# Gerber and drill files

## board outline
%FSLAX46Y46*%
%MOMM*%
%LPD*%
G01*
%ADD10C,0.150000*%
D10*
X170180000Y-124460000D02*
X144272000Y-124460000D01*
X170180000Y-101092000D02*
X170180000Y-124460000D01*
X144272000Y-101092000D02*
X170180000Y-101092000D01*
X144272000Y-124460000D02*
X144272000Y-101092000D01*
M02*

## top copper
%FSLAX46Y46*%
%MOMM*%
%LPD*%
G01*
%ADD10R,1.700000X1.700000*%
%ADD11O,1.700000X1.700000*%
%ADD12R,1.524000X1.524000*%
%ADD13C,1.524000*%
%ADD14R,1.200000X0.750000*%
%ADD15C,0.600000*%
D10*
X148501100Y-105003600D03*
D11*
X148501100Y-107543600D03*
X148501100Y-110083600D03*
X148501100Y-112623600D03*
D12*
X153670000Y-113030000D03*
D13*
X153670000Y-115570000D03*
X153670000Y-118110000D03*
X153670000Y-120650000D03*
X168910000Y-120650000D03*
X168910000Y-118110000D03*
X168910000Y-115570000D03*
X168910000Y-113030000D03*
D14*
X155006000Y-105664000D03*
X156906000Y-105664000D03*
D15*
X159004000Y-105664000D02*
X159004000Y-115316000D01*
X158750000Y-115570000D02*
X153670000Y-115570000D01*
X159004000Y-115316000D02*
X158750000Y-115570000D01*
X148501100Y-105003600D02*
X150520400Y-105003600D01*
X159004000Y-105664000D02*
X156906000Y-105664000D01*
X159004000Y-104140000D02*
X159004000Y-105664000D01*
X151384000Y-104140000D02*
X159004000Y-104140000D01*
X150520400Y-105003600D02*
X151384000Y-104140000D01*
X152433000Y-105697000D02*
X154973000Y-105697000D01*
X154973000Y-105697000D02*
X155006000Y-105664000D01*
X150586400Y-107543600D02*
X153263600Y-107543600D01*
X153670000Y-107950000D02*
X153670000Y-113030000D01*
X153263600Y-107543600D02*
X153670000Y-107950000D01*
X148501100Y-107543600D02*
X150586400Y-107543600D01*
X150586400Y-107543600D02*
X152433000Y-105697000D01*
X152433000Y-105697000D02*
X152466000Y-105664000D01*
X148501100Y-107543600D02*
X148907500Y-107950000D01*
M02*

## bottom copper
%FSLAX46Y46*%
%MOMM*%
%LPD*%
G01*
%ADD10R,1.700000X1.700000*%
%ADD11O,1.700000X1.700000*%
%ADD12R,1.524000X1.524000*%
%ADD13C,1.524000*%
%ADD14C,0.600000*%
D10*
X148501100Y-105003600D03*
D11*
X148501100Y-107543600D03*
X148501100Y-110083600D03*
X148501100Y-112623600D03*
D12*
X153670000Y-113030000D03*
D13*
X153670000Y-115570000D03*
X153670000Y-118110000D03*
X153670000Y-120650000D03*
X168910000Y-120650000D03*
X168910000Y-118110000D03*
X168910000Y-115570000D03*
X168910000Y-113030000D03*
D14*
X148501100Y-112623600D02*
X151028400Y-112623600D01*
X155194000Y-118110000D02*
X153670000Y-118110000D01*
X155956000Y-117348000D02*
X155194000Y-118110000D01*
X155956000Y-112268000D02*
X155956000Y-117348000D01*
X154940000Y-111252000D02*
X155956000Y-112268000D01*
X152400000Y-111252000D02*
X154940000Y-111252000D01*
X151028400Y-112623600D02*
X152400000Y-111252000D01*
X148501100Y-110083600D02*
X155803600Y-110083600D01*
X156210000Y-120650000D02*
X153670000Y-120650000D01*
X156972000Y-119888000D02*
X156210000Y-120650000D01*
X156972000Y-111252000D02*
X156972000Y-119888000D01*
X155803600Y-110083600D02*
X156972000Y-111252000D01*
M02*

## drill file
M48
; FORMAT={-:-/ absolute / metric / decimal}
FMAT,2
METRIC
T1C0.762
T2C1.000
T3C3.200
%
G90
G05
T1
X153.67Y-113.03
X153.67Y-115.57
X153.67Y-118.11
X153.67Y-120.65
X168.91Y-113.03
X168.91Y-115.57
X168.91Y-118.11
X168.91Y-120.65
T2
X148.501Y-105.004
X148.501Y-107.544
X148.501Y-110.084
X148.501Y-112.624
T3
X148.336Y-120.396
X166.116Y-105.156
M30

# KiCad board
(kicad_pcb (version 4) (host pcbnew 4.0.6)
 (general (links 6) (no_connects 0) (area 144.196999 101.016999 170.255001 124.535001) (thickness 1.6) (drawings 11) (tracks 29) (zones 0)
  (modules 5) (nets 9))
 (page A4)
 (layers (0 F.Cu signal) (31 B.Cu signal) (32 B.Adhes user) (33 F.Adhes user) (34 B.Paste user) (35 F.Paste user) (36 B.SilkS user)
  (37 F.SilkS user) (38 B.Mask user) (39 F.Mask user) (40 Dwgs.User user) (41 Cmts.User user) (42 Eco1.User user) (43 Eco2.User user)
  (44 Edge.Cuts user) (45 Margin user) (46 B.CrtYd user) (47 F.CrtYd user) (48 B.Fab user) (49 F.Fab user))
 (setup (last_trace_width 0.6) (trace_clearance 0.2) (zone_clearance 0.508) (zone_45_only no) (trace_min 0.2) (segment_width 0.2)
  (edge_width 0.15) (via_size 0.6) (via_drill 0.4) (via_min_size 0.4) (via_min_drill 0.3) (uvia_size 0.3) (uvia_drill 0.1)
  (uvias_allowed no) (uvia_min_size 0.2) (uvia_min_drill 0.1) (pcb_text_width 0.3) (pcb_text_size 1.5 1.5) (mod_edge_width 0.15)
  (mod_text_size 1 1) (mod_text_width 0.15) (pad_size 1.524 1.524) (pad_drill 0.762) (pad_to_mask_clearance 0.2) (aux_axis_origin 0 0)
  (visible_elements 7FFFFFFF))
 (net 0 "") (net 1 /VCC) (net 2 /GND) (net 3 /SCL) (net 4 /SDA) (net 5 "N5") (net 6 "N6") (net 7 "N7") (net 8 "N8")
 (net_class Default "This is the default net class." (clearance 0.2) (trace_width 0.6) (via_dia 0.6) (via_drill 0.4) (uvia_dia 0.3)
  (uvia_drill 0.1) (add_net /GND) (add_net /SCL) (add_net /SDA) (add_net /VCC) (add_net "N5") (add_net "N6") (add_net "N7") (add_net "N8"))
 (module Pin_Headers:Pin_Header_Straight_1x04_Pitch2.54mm (layer F.Cu) (at 148.5011 105.0036)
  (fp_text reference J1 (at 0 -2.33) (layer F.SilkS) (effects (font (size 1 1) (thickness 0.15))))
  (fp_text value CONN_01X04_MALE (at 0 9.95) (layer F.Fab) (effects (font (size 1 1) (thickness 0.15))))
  (pad 1 thru_hole rect (at 0 0) (size 1.7 1.7) (drill 1) (layers *.Cu *.Mask) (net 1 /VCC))
  (pad 2 thru_hole oval (at 0 2.54) (size 1.7 1.7) (drill 1) (layers *.Cu *.Mask) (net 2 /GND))
  (pad 3 thru_hole oval (at 0 5.08) (size 1.7 1.7) (drill 1) (layers *.Cu *.Mask) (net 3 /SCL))
  (pad 4 thru_hole oval (at 0 7.62) (size 1.7 1.7) (drill 1) (layers *.Cu *.Mask) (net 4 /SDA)))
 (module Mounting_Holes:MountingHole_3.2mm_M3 (layer F.Cu) (at 148.336 120.396)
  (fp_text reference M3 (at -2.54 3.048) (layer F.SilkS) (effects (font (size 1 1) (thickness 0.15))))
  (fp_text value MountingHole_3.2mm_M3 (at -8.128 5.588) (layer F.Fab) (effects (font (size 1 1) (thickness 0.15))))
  (pad 1 np_thru_hole circle (at 0 0) (size 3.2 3.2) (drill 3.2) (layers *.Cu *.Mask)))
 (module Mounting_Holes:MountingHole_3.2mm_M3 (layer F.Cu) (at 166.116 105.156)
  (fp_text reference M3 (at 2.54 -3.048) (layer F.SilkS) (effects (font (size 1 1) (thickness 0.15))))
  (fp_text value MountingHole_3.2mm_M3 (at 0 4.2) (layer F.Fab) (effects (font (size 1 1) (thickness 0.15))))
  (pad 1 np_thru_hole circle (at 0 0) (size 3.2 3.2) (drill 3.2) (layers *.Cu *.Mask)))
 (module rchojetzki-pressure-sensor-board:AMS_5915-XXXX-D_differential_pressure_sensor (layer F.Cu) (at 153.67 109.22 270)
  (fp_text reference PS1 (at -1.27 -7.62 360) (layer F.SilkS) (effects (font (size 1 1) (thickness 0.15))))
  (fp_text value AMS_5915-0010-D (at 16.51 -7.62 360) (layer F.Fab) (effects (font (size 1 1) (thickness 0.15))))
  (pad 1 thru_hole rect (at 3.81 0 270) (size 1.524 1.524) (drill 0.762) (layers *.Cu *.Mask) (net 2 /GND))
  (pad 2 thru_hole circle (at 6.35 0 270) (size 1.524 1.524) (drill 0.762) (layers *.Cu *.Mask) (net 1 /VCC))
  (pad 3 thru_hole circle (at 8.89 0 270) (size 1.524 1.524) (drill 0.762) (layers *.Cu *.Mask) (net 4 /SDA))
  (pad 4 thru_hole circle (at 11.43 0 270) (size 1.524 1.524) (drill 0.762) (layers *.Cu *.Mask) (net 3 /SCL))
  (pad 5 thru_hole circle (at 11.43 -15.24 270) (size 1.524 1.524) (drill 0.762) (layers *.Cu *.Mask) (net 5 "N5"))
  (pad 6 thru_hole circle (at 8.89 -15.24 270) (size 1.524 1.524) (drill 0.762) (layers *.Cu *.Mask) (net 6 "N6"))
  (pad 7 thru_hole circle (at 6.35 -15.24 270) (size 1.524 1.524) (drill 0.762) (layers *.Cu *.Mask) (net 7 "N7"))
  (pad 8 thru_hole circle (at 3.81 -15.24 270) (size 1.524 1.524) (drill 0.762) (layers *.Cu *.Mask) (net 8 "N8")))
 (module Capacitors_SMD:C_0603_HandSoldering (layer F.Cu) (at 155.956 105.664)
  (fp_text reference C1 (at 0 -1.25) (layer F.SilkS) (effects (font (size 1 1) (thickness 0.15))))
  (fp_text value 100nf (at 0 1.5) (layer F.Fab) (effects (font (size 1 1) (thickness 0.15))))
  (pad 1 smd rect (at -0.95 0) (size 1.2 0.75) (layers F.Cu F.Paste F.Mask) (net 2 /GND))
  (pad 2 smd rect (at 0.95 0) (size 1.2 0.75) (layers F.Cu F.Paste F.Mask) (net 1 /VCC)))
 (gr_line (start 170.18 124.46) (end 144.272 124.46) (angle 90) (layer Edge.Cuts) (width 0.15))
 (gr_line (start 170.18 101.092) (end 170.18 124.46) (angle 90) (layer Edge.Cuts) (width 0.15))
 (gr_line (start 144.272 101.092) (end 170.18 101.092) (angle 90) (layer Edge.Cuts) (width 0.15))
 (gr_line (start 144.272 124.46) (end 144.272 101.092) (angle 90) (layer Edge.Cuts) (width 0.15))
 (segment (start 159.004 105.664) (end 159.004 115.316) (width 0.6) (layer F.Cu) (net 1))
 (segment (start 158.75 115.57) (end 153.67 115.57) (width 0.6) (layer F.Cu) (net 1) (status 800000))
 (segment (start 159.004 115.316) (end 158.75 115.57) (width 0.6) (layer F.Cu) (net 1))
 (segment (start 148.5011 105.0036) (end 150.5204 105.0036) (width 0.6) (layer F.Cu) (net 1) (status 400000))
 (segment (start 159.004 105.664) (end 156.906 105.664) (width 0.6) (layer F.Cu) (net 1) (status 800000))
 (segment (start 159.004 104.14) (end 159.004 105.664) (width 0.6) (layer F.Cu) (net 1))
 (segment (start 151.384 104.14) (end 159.004 104.14) (width 0.6) (layer F.Cu) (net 1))
 (segment (start 150.5204 105.0036) (end 151.384 104.14) (width 0.6) (layer F.Cu) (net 1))
 (segment (start 152.433 105.697) (end 154.973 105.697) (width 0.6) (layer F.Cu) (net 2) (status 800000))
 (segment (start 154.973 105.697) (end 155.006 105.664) (width 0.6) (layer F.Cu) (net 2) (status C00000))
 (segment (start 150.5864 107.5436) (end 153.2636 107.5436) (width 0.6) (layer F.Cu) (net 2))
 (segment (start 153.67 107.95) (end 153.67 113.03) (width 0.6) (layer F.Cu) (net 2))
 (segment (start 153.2636 107.5436) (end 153.67 107.95) (width 0.6) (layer F.Cu) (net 2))
 (segment (start 148.5011 107.5436) (end 150.5864 107.5436) (width 0.6) (layer F.Cu) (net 2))
 (segment (start 150.5864 107.5436) (end 152.433 105.697) (width 0.6) (layer F.Cu) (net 2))
 (segment (start 152.433 105.697) (end 152.466 105.664) (width 0.6) (layer F.Cu) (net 2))
 (segment (start 148.5011 107.5436) (end 148.9075 107.95) (width 0.6) (layer F.Cu) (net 2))
 (segment (start 148.5011 112.6236) (end 151.0284 112.6236) (width 0.6) (layer B.Cu) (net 4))
 (segment (start 155.194 118.11) (end 153.67 118.11) (width 0.6) (layer B.Cu) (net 4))
 (segment (start 155.956 117.348) (end 155.194 118.11) (width 0.6) (layer B.Cu) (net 4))
 (segment (start 155.956 112.268) (end 155.956 117.348) (width 0.6) (layer B.Cu) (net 4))
 (segment (start 154.94 111.252) (end 155.956 112.268) (width 0.6) (layer B.Cu) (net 4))
 (segment (start 152.4 111.252) (end 154.94 111.252) (width 0.6) (layer B.Cu) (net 4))
 (segment (start 151.0284 112.6236) (end 152.4 111.252) (width 0.6) (layer B.Cu) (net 4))
 (segment (start 148.5011 110.0836) (end 155.8036 110.0836) (width 0.6) (layer B.Cu) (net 3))
 (segment (start 156.21 120.65) (end 153.67 120.65) (width 0.6) (layer B.Cu) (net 3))
 (segment (start 156.972 119.888) (end 156.21 120.65) (width 0.6) (layer B.Cu) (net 3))
 (segment (start 156.972 111.252) (end 156.972 119.888) (width 0.6) (layer B.Cu) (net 3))
 (segment (start 155.8036 110.0836) (end 156.972 111.252) (width 0.6) (layer B.Cu) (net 3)))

